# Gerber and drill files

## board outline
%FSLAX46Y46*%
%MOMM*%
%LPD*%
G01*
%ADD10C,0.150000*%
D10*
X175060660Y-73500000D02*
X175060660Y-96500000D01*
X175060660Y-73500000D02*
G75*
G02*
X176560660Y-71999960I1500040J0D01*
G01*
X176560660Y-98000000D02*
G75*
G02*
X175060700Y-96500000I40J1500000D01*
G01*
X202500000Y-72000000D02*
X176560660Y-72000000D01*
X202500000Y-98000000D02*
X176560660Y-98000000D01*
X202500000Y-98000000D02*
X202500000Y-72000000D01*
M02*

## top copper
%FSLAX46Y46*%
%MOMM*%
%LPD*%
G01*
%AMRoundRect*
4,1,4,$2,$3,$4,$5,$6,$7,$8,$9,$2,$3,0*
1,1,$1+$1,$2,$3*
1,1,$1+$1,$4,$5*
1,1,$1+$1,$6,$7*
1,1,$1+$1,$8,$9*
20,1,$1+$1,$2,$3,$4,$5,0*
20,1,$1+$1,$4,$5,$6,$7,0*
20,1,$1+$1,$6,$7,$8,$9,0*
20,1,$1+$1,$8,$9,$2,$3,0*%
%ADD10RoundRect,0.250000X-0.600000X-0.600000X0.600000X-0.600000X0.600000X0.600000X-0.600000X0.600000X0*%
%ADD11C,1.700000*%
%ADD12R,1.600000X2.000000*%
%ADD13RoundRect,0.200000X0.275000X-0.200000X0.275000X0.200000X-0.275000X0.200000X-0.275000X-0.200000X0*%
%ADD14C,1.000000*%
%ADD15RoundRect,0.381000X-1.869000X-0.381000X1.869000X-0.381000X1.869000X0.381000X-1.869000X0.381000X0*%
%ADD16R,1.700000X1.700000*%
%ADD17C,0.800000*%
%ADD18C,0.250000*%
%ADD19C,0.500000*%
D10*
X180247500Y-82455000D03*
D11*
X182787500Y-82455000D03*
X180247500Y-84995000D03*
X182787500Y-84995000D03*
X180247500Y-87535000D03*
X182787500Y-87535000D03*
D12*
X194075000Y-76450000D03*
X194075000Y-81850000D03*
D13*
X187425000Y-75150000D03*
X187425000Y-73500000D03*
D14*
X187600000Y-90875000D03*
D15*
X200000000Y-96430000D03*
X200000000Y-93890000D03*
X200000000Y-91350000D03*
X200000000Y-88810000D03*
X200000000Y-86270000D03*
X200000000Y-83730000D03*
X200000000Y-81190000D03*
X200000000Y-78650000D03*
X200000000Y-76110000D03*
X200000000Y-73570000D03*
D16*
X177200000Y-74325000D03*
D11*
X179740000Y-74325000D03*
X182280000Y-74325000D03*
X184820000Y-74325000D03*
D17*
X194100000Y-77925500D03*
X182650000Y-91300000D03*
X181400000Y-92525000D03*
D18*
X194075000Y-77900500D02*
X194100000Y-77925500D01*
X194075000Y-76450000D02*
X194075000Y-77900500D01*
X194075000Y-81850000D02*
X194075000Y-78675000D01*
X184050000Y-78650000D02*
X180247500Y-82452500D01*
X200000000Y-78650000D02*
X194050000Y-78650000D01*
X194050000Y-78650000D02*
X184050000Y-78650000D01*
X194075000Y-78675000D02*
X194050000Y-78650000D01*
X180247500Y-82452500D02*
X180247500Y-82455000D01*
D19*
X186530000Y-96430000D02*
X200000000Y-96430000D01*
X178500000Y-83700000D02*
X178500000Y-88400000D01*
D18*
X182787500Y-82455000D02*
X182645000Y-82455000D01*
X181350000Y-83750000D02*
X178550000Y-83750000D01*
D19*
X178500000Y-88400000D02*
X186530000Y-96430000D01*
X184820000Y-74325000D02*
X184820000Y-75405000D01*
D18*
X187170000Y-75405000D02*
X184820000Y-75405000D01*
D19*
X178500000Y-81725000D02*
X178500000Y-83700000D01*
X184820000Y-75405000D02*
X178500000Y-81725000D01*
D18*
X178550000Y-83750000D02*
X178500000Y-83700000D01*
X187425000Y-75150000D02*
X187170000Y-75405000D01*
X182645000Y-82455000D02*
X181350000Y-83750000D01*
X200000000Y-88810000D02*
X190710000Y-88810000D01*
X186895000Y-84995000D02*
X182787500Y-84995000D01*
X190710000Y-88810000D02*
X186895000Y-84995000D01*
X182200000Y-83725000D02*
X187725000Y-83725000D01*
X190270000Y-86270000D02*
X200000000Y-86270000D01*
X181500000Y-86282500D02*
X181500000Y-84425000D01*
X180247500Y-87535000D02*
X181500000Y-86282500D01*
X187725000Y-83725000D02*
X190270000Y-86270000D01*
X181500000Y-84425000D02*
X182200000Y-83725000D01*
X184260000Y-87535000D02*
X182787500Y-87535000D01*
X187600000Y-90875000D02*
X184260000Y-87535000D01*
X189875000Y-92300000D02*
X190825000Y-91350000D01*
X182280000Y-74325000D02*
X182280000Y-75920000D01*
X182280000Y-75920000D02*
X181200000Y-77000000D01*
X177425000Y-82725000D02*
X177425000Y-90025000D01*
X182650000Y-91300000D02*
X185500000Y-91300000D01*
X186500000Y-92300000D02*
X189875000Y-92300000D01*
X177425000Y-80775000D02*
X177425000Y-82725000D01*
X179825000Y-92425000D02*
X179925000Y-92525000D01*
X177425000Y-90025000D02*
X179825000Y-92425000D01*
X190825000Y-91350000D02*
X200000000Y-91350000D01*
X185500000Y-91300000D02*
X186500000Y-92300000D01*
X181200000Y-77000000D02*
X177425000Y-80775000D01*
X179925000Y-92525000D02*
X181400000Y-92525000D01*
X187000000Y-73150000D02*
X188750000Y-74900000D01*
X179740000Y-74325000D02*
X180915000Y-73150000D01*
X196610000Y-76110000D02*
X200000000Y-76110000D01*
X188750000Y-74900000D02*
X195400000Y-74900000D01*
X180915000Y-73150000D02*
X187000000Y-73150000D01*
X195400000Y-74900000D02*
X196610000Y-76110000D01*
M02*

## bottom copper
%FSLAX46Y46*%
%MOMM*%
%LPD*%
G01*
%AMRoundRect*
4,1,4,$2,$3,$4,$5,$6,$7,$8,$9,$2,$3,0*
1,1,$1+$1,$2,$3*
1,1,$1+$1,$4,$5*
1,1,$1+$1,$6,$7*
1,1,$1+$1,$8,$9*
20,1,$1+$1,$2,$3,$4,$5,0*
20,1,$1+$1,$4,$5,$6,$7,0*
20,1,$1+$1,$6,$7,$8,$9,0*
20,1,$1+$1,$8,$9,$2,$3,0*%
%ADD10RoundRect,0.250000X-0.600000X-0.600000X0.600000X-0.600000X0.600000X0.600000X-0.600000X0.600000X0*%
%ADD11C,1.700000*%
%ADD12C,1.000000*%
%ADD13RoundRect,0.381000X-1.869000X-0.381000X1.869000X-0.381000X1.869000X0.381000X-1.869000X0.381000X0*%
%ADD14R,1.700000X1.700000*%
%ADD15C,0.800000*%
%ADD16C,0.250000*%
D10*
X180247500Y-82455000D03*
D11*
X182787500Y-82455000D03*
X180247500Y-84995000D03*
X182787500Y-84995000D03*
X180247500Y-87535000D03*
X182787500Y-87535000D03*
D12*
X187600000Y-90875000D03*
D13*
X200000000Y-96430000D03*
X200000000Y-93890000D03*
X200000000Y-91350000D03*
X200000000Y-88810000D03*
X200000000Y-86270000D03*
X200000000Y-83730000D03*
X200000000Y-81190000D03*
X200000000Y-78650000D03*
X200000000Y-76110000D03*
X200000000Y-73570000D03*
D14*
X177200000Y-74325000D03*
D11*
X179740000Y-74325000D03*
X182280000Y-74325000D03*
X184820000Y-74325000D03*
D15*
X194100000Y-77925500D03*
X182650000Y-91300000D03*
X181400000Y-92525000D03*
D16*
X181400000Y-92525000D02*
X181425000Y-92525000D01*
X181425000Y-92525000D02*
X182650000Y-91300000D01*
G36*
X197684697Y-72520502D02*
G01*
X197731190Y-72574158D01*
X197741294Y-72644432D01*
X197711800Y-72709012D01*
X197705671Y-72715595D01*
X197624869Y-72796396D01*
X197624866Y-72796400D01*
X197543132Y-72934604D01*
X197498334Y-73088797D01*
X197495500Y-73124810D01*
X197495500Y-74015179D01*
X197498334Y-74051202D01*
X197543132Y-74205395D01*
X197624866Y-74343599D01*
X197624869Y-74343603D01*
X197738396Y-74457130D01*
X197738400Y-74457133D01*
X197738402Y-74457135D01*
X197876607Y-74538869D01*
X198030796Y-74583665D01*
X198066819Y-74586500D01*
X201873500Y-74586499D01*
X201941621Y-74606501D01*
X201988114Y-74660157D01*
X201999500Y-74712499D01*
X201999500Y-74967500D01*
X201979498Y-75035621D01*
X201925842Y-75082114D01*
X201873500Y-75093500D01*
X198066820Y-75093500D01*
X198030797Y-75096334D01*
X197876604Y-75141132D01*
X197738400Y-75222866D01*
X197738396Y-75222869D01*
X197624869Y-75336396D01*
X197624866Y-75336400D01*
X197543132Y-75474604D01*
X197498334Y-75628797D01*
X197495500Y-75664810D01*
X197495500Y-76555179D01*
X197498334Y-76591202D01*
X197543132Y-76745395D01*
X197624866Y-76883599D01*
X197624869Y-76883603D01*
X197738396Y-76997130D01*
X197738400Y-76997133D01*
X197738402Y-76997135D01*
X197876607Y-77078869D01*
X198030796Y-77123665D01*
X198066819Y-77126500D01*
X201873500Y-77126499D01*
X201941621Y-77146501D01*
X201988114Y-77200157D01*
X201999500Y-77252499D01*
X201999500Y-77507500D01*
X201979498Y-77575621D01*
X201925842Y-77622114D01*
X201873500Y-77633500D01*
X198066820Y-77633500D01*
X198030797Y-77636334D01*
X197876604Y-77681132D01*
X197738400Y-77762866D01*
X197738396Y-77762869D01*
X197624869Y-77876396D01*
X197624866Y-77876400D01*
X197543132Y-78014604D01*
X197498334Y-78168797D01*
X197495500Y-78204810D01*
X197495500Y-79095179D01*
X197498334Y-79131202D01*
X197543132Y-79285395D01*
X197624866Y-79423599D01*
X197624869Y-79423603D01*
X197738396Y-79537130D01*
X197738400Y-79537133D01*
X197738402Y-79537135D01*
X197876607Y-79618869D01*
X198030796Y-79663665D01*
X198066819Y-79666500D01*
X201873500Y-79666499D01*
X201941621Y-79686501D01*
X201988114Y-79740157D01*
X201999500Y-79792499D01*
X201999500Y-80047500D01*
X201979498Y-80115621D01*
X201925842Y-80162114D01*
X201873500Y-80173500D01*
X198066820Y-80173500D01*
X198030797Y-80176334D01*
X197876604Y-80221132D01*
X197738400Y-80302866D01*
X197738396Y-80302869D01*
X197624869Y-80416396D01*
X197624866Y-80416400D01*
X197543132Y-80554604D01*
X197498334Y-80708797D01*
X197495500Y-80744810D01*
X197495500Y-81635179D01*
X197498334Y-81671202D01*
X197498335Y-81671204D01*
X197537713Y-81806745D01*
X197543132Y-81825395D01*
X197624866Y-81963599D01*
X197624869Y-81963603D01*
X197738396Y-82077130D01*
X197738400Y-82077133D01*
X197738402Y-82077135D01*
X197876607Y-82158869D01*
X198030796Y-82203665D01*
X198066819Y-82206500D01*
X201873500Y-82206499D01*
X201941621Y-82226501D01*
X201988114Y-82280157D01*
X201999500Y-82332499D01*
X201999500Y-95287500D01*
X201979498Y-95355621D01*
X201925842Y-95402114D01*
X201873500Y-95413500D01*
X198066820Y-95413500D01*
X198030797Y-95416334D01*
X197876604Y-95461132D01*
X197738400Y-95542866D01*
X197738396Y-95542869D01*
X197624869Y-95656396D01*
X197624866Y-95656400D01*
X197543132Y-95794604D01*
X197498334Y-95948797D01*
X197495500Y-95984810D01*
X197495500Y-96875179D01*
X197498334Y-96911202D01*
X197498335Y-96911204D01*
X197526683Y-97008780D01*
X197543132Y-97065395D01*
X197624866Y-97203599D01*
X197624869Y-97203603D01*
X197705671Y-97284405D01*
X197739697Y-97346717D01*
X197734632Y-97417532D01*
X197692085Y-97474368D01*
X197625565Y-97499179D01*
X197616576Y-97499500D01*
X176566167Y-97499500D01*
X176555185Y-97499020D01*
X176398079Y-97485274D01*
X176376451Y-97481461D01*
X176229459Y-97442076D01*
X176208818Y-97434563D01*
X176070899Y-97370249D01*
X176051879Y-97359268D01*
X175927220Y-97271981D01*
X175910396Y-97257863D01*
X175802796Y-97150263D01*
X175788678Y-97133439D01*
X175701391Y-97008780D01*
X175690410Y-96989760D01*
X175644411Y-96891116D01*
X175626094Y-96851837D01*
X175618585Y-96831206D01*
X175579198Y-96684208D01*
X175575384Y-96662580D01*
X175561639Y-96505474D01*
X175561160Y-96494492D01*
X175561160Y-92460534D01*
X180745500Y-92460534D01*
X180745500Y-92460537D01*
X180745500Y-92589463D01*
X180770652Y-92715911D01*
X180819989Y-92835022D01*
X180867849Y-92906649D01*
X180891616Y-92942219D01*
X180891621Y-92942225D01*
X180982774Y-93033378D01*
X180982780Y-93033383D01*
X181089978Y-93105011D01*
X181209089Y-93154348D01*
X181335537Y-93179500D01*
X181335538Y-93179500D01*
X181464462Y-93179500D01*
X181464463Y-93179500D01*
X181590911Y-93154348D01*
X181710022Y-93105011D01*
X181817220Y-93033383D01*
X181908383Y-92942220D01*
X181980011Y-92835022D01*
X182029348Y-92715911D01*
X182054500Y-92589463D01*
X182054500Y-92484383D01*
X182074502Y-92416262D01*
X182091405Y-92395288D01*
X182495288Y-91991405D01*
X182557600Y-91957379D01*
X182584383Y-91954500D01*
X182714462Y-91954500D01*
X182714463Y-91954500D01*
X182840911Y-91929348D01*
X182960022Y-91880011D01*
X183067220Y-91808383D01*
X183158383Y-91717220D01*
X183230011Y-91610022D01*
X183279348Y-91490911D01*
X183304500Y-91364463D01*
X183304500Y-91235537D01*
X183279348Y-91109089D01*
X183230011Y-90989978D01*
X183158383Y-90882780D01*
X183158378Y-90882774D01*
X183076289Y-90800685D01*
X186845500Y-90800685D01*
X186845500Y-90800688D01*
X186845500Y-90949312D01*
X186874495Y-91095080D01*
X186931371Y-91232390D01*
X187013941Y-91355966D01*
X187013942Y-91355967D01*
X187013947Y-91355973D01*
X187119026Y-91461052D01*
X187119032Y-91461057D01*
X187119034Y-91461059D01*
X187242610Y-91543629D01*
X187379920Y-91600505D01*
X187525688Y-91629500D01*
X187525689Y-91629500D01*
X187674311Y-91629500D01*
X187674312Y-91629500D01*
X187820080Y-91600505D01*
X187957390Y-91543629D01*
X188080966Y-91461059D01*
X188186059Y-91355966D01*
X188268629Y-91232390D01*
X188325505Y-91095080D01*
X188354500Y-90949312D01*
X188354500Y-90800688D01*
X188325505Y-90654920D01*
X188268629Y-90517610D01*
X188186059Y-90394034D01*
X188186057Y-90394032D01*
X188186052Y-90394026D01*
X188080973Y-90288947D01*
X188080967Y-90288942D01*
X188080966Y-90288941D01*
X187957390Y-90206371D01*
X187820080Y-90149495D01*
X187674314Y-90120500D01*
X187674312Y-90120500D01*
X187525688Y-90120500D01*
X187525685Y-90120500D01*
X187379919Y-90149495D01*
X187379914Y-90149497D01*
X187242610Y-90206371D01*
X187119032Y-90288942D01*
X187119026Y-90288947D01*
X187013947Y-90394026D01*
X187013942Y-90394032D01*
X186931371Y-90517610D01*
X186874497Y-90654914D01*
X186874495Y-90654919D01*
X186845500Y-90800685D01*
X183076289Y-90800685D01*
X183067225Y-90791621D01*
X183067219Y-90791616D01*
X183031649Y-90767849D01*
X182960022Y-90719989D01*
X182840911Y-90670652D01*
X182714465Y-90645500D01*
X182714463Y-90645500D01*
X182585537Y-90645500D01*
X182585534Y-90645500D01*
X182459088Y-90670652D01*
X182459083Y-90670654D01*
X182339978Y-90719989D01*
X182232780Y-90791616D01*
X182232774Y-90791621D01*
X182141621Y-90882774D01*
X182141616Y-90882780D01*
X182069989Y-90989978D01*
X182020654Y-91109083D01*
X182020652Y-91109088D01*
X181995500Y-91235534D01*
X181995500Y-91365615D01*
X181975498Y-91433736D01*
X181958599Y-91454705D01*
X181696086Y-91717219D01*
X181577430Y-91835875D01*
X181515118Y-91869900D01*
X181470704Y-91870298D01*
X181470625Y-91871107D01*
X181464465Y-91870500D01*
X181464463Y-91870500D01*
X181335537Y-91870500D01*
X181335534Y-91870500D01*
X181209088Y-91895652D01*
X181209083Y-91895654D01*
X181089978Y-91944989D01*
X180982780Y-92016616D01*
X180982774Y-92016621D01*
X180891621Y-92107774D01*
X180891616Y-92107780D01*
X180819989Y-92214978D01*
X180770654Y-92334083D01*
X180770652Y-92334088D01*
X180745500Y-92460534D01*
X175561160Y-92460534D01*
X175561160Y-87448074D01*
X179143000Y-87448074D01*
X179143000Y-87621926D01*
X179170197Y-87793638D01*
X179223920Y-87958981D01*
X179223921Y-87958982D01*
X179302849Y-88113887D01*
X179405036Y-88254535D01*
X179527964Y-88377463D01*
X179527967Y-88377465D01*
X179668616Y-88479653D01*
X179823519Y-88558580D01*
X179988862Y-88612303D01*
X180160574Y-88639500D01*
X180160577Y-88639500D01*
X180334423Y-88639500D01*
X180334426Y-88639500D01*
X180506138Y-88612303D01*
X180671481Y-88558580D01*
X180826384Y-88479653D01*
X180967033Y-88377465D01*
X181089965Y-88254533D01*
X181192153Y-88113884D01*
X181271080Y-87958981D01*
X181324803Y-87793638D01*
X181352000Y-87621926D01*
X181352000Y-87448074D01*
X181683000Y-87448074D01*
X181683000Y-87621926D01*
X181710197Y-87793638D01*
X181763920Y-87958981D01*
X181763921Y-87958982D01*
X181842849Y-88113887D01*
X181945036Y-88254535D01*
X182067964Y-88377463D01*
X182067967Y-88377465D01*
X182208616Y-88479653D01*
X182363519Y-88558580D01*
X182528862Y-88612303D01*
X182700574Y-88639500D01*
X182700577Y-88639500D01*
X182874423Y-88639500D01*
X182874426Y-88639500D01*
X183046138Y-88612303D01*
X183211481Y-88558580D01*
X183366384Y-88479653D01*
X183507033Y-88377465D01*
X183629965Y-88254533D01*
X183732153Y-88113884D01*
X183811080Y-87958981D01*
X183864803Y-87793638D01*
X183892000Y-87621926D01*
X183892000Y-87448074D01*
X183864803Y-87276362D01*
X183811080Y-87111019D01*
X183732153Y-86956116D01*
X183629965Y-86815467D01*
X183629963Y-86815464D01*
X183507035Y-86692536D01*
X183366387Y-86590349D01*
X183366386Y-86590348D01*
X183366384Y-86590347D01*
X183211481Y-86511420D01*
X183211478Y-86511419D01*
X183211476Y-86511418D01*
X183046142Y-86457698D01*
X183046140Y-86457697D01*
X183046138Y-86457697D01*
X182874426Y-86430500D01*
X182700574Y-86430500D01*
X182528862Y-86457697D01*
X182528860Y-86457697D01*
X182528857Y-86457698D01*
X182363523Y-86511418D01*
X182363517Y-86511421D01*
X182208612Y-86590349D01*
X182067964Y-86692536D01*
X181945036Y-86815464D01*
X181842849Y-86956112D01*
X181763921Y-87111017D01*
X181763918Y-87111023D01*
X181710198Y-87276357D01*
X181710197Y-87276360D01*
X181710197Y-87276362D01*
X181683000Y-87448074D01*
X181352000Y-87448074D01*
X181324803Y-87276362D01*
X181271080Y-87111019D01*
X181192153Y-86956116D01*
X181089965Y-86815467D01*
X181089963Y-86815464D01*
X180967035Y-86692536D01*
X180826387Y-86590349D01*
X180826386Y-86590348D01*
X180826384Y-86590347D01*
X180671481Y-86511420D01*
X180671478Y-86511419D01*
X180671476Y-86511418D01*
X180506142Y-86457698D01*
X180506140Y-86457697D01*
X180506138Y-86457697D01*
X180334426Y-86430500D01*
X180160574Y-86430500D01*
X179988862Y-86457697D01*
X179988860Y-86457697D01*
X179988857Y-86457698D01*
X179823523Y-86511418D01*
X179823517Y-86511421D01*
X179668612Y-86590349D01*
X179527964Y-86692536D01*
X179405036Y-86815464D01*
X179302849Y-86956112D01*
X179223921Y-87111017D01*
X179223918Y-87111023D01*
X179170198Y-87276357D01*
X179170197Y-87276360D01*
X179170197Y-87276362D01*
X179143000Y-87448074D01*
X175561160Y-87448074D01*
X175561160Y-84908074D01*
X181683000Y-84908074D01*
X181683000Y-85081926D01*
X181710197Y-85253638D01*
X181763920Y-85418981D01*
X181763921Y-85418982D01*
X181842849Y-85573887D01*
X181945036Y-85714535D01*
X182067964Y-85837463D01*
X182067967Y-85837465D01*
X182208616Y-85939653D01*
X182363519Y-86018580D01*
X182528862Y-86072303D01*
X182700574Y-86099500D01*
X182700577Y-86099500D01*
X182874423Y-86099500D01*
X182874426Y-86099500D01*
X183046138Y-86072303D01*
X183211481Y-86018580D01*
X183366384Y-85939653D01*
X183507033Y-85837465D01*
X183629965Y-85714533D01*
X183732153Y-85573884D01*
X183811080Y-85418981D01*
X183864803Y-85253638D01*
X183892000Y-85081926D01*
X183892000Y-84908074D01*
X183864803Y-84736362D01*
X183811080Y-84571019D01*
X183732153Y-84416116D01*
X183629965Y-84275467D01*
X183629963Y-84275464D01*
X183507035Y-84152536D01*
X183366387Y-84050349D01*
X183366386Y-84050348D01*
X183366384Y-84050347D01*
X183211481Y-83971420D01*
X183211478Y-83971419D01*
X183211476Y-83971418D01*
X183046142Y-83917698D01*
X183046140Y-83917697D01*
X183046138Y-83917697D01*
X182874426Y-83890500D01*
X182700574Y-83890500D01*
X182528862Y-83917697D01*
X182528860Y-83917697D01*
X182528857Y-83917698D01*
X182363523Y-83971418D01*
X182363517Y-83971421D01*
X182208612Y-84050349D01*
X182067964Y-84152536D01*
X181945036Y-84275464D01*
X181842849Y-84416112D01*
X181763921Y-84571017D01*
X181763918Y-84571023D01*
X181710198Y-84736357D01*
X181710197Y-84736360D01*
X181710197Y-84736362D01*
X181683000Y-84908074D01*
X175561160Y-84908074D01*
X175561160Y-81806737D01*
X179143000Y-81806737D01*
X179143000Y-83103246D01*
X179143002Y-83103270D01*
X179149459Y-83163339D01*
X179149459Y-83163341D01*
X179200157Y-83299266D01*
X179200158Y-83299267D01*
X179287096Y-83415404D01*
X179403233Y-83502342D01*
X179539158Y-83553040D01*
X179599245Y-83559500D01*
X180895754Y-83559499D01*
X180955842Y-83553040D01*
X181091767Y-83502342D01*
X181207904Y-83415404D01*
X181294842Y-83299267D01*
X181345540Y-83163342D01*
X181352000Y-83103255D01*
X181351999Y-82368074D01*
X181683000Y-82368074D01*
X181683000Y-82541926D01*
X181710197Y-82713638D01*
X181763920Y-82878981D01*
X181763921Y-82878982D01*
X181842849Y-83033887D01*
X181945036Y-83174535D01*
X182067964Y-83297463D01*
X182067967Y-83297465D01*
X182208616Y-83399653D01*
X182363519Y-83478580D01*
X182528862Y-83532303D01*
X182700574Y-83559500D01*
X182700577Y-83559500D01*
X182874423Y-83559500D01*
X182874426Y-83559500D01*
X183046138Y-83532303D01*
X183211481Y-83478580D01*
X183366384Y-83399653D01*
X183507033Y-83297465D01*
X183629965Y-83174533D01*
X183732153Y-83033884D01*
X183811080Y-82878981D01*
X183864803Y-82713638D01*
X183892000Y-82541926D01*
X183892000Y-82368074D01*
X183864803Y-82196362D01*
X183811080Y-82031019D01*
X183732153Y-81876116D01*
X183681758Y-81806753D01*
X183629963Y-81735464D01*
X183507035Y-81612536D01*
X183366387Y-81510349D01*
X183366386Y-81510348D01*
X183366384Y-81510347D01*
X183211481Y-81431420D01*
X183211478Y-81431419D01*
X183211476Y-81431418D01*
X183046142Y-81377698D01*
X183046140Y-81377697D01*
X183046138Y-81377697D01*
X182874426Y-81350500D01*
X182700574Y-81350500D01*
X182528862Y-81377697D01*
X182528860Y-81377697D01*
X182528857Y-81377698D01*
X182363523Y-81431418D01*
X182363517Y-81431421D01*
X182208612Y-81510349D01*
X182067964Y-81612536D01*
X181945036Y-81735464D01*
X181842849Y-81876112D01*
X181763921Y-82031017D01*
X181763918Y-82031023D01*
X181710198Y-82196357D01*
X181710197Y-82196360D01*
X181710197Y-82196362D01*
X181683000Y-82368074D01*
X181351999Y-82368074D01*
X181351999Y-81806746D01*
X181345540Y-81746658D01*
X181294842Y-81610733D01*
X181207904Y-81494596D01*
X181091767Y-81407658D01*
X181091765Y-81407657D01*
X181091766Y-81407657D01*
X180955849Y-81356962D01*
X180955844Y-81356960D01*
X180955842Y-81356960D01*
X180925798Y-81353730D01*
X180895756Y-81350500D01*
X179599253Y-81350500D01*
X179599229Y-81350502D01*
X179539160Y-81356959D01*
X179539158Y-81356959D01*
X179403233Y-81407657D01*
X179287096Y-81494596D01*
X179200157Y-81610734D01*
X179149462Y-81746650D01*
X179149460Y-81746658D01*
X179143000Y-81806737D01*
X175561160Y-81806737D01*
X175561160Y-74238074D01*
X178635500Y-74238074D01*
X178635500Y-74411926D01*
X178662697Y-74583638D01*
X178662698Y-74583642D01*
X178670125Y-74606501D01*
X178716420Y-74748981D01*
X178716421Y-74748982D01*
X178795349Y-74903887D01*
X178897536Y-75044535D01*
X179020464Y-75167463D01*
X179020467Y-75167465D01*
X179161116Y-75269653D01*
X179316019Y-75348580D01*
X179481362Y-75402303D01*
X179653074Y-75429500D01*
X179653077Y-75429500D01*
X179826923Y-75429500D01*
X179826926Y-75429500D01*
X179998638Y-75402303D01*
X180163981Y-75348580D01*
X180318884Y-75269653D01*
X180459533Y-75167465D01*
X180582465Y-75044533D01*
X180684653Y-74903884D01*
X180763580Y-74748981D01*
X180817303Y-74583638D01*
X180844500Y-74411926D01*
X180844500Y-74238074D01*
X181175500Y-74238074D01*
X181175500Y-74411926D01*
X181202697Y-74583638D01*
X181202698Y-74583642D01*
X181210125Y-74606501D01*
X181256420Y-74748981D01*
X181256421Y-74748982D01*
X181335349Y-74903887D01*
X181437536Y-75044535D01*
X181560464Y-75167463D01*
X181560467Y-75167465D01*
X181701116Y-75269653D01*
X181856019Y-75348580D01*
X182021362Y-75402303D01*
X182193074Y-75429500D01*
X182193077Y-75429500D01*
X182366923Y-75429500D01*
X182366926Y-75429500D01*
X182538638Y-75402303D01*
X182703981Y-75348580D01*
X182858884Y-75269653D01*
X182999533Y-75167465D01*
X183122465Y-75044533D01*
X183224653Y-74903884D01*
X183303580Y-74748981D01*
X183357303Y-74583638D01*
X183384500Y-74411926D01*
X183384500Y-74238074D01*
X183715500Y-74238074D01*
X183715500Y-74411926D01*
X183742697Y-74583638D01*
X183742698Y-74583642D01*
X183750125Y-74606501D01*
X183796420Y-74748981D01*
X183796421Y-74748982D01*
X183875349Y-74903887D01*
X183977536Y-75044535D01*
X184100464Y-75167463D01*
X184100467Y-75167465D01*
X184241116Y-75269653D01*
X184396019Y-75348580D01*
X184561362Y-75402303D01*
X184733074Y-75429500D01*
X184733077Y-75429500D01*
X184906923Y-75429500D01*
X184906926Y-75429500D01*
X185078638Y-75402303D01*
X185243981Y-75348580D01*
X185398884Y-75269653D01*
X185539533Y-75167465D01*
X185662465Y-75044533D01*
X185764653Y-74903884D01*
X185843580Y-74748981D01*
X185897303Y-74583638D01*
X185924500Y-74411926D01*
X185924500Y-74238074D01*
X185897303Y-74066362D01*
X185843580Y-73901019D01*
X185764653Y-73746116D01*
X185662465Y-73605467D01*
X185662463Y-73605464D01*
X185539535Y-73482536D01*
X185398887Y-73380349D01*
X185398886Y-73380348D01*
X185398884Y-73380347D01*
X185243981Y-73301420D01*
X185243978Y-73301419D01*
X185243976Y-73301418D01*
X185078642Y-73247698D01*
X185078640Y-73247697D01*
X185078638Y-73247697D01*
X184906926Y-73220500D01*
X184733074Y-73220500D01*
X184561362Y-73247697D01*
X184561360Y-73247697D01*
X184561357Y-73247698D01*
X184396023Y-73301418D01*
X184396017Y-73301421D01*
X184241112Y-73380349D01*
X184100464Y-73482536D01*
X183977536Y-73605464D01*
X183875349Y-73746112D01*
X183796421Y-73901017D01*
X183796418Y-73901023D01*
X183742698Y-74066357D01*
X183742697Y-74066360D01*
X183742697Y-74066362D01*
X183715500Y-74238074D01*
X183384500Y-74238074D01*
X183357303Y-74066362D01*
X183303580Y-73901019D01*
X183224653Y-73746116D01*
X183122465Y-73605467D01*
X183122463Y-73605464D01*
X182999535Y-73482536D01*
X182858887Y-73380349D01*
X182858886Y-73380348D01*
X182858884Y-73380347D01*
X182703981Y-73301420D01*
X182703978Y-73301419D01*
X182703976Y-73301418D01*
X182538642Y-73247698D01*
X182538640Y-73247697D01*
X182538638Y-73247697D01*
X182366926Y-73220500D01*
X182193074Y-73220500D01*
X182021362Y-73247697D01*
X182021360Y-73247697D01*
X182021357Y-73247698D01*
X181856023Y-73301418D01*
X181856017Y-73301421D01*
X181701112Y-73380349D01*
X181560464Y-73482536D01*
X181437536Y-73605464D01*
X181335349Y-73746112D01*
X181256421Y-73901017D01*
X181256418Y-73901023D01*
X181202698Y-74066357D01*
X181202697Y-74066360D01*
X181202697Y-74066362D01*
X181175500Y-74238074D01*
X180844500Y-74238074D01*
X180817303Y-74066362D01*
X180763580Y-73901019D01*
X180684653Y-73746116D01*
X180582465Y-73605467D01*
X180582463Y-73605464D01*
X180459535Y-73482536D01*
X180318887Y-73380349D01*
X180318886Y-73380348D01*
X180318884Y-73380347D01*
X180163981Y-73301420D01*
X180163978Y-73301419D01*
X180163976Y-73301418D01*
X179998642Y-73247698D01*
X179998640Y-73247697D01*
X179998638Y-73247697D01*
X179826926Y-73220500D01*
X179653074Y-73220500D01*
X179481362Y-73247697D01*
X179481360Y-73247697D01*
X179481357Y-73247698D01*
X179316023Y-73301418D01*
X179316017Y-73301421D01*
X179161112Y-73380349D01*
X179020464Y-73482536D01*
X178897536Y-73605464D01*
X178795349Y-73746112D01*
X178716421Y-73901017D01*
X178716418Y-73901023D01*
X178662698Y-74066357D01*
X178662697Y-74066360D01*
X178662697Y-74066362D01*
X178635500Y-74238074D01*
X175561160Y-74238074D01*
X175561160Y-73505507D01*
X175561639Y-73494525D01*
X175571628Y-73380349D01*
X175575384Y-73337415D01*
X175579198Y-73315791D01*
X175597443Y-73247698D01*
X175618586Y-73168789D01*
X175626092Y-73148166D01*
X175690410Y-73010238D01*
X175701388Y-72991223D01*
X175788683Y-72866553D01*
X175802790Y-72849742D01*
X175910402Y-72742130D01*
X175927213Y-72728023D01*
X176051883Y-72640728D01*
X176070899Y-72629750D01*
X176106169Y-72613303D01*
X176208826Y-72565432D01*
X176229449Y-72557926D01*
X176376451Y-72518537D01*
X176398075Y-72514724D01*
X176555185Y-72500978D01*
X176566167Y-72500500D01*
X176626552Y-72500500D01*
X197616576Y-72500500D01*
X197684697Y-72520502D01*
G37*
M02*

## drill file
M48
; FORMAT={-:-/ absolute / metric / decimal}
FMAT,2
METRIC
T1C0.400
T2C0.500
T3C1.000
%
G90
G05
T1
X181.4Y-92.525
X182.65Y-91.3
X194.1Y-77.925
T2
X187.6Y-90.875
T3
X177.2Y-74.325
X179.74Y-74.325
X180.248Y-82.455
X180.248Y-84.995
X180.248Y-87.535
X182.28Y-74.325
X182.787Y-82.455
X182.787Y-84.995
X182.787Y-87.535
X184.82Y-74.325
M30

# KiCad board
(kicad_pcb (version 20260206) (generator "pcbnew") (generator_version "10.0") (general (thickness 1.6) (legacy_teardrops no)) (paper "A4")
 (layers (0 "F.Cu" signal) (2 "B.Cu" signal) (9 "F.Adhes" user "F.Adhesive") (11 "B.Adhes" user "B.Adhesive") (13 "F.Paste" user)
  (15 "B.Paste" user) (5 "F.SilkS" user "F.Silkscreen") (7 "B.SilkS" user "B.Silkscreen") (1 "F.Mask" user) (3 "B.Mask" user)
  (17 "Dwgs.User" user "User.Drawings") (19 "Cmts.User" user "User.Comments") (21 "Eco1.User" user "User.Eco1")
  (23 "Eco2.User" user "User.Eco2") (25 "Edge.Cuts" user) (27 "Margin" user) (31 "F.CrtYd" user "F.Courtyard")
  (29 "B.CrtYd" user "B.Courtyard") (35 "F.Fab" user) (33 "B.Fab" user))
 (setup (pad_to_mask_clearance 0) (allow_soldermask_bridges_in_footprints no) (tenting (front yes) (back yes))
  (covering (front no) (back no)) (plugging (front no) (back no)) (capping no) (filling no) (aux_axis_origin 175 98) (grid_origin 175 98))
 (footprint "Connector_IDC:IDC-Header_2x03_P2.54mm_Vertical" (layer "F.Cu") (at 180.2475 82.455)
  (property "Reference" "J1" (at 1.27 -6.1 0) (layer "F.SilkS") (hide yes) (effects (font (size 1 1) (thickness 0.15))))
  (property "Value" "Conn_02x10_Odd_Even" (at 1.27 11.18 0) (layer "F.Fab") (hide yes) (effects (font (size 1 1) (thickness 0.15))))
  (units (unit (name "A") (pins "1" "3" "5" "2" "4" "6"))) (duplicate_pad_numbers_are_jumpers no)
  (pad "1" thru_hole roundrect (at 0 0) (size 1.7 1.7) (drill 1) (layers "*.Cu" "*.Mask") (remove_unused_layers no)
   (roundrect_rratio 0.147059) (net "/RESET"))
  (pad "2" thru_hole circle (at 2.54 0) (size 1.7 1.7) (drill 1) (layers "*.Cu" "*.Mask") (remove_unused_layers no) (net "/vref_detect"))
  (pad "3" thru_hole circle (at 0 2.54) (size 1.7 1.7) (drill 1) (layers "*.Cu" "*.Mask") (remove_unused_layers no) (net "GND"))
  (pad "4" thru_hole circle (at 2.54 2.54) (size 1.7 1.7) (drill 1) (layers "*.Cu" "*.Mask") (remove_unused_layers no) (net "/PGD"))
  (pad "5" thru_hole circle (at 0 5.08) (size 1.7 1.7) (drill 1) (layers "*.Cu" "*.Mask") (remove_unused_layers no) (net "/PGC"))
  (pad "6" thru_hole circle (at 2.54 5.08) (size 1.7 1.7) (drill 1) (layers "*.Cu" "*.Mask") (remove_unused_layers no) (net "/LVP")))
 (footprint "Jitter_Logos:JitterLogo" (layer "F.Cu") (at 193.607667 90.975)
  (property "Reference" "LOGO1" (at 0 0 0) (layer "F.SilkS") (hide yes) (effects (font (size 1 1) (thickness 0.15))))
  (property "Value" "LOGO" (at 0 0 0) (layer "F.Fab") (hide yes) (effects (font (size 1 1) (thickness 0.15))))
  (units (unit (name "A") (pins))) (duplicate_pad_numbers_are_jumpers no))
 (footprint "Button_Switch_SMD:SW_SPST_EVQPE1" (layer "F.Cu") (at 194.075 79.15 -90)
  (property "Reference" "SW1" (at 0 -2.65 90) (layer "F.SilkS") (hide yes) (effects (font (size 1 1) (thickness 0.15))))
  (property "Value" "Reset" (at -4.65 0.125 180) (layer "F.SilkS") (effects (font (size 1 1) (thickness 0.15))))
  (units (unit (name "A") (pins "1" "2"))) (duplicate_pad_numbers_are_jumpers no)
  (pad "1" smd rect (at -2.7 0 270) (size 2 1.6) (layers "F.Cu" "F.Mask" "F.Paste") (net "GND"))
  (pad "2" smd rect (at 2.7 0 270) (size 2 1.6) (layers "F.Cu" "F.Mask" "F.Paste") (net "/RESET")))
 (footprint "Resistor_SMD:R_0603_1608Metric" (layer "F.Cu") (at 187.425 74.325 90)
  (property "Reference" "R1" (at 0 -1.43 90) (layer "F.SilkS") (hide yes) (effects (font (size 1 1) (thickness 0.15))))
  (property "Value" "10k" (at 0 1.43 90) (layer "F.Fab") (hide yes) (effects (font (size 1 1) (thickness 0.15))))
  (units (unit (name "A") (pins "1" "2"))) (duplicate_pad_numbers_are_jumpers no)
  (pad "1" smd roundrect (at -0.825 0 90) (size 0.8 0.95) (layers "F.Cu" "F.Mask" "F.Paste") (roundrect_rratio 0.25) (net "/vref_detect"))
  (pad "2" smd roundrect (at 0.825 0 90) (size 0.8 0.95) (layers "F.Cu" "F.Mask" "F.Paste") (roundrect_rratio 0.25) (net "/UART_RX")))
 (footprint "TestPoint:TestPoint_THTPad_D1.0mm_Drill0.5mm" (layer "F.Cu") (at 187.6 90.875)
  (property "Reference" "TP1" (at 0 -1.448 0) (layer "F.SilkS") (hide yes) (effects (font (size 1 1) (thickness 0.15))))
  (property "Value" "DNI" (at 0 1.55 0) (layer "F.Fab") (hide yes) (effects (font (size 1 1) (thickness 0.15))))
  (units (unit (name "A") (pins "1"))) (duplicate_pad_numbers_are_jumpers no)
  (pad "1" thru_hole circle (at 0 0) (size 1 1) (drill 0.5) (layers "*.Cu" "*.Mask") (remove_unused_layers no) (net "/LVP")))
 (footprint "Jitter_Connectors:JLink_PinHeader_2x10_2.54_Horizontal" (layer "F.Cu") (at 200 85)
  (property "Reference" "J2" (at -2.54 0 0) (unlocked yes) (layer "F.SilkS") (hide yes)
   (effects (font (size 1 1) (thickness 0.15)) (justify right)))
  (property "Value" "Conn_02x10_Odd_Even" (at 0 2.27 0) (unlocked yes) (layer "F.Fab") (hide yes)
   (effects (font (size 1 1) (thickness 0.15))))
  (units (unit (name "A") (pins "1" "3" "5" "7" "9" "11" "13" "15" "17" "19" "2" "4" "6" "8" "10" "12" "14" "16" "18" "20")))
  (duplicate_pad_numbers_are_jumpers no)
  (pad "1" smd roundrect (at 0 11.43) (size 4.5 1.524) (layers "F.Cu" "F.Mask" "F.Paste") (roundrect_rratio 0.25) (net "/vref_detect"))
  (pad "2" smd roundrect (at 0 11.43) (size 4.5 1.524) (layers "B.Cu" "B.Mask" "B.Paste") (roundrect_rratio 0.25)
   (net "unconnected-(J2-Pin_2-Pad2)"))
  (pad "3" smd roundrect (at 0 8.89) (size 4.5 1.524) (layers "F.Cu" "F.Mask" "F.Paste") (roundrect_rratio 0.25)
   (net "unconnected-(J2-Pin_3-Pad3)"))
  (pad "4" smd roundrect (at 0 8.89) (size 4.5 1.524) (layers "B.Cu" "B.Mask" "B.Paste") (roundrect_rratio 0.25) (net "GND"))
  (pad "5" smd roundrect (at 0 6.35) (size 4.5 1.524) (layers "F.Cu" "F.Mask" "F.Paste") (roundrect_rratio 0.25) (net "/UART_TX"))
  (pad "6" smd roundrect (at 0 6.35) (size 4.5 1.524) (layers "B.Cu" "B.Mask" "B.Paste") (roundrect_rratio 0.25) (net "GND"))
  (pad "7" smd roundrect (at 0 3.81) (size 4.5 1.524) (layers "F.Cu" "F.Mask" "F.Paste") (roundrect_rratio 0.25) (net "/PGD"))
  (pad "8" smd roundrect (at 0 3.81) (size 4.5 1.524) (layers "B.Cu" "B.Mask" "B.Paste") (roundrect_rratio 0.25) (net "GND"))
  (pad "9" smd roundrect (at 0 1.27) (size 4.5 1.524) (layers "F.Cu" "F.Mask" "F.Paste") (roundrect_rratio 0.25) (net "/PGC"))
  (pad "10" smd roundrect (at 0 1.27) (size 4.5 1.524) (layers "B.Cu" "B.Mask" "B.Paste") (roundrect_rratio 0.25) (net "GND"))
  (pad "11" smd roundrect (at 0 -1.27) (size 4.5 1.524) (layers "F.Cu" "F.Mask" "F.Paste") (roundrect_rratio 0.25)
   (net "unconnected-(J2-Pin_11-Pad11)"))
  (pad "12" smd roundrect (at 0 -1.27) (size 4.5 1.524) (layers "B.Cu" "B.Mask" "B.Paste") (roundrect_rratio 0.25) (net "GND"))
  (pad "13" smd roundrect (at 0 -3.81) (size 4.5 1.524) (layers "F.Cu" "F.Mask" "F.Paste") (roundrect_rratio 0.25)
   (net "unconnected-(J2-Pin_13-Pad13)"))
  (pad "14" smd roundrect (at 0 -3.81) (size 4.5 1.524) (layers "B.Cu" "B.Mask" "B.Paste") (roundrect_rratio 0.25)
   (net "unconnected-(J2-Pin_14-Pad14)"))
  (pad "15" smd roundrect (at 0 -6.35) (size 4.5 1.524) (layers "F.Cu" "F.Mask" "F.Paste") (roundrect_rratio 0.25) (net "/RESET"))
  (pad "16" smd roundrect (at 0 -6.35) (size 4.5 1.524) (layers "B.Cu" "B.Mask" "B.Paste") (roundrect_rratio 0.25)
   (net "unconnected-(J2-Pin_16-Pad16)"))
  (pad "17" smd roundrect (at 0 -8.89) (size 4.5 1.524) (layers "F.Cu" "F.Mask" "F.Paste") (roundrect_rratio 0.25) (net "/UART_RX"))
  (pad "18" smd roundrect (at 0 -8.89) (size 4.5 1.524) (layers "B.Cu" "B.Mask" "B.Paste") (roundrect_rratio 0.25)
   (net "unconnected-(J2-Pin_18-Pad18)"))
  (pad "19" smd roundrect (at 0 -11.43) (size 4.5 1.524) (layers "F.Cu" "F.Mask" "F.Paste") (roundrect_rratio 0.25)
   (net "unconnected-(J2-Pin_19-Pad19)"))
  (pad "20" smd roundrect (at 0 -11.43) (size 4.5 1.524) (layers "B.Cu" "B.Mask" "B.Paste") (roundrect_rratio 0.25)
   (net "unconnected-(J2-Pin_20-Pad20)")))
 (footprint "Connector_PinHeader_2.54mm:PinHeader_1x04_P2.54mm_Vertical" (layer "F.Cu") (at 177.2 74.325 90)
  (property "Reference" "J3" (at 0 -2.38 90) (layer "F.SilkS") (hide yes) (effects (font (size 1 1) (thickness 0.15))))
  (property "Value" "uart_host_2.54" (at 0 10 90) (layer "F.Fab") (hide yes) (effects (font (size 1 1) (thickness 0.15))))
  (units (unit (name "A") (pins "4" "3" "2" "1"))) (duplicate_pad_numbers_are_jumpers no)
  (pad "1" thru_hole rect (at 0 0 90) (size 1.7 1.7) (drill 1) (layers "*.Cu" "*.Mask") (remove_unused_layers no) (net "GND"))
  (pad "2" thru_hole circle (at 0 2.54 90) (size 1.7 1.7) (drill 1) (layers "*.Cu" "*.Mask") (remove_unused_layers no) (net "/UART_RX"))
  (pad "3" thru_hole circle (at 0 5.08 90) (size 1.7 1.7) (drill 1) (layers "*.Cu" "*.Mask") (remove_unused_layers no) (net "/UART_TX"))
  (pad "4" thru_hole circle (at 0 7.62 90) (size 1.7 1.7) (drill 1) (layers "*.Cu" "*.Mask") (remove_unused_layers no) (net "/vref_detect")))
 (gr_line (start 175.06066 73.5) (end 175.06066 96.5) (stroke (width 0.15) (type solid)) (layer "Edge.Cuts"))
 (gr_arc (start 175.06066 73.5) (mid 175.5 72.43934) (end 176.56066 72) (stroke (width 0.15) (type solid)) (layer "Edge.Cuts"))
 (gr_arc (start 176.56066 98) (mid 175.5 97.56066) (end 175.06066 96.5) (stroke (width 0.15) (type solid)) (layer "Edge.Cuts"))
 (gr_line (start 202.5 72) (end 176.56066 72) (stroke (width 0.15) (type solid)) (layer "Edge.Cuts"))
 (gr_line (start 202.5 98) (end 176.56066 98) (stroke (width 0.15) (type solid)) (layer "Edge.Cuts"))
 (gr_line (start 202.5 98) (end 202.5 72) (stroke (width 0.15) (type solid)) (layer "Edge.Cuts"))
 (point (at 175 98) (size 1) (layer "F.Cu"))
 (segment (start 194.075 77.9005) (end 194.1 77.9255) (width 0.25) (layer "F.Cu") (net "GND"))
 (segment (start 194.075 76.45) (end 194.075 77.9005) (width 0.25) (layer "F.Cu") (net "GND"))
 (via (at 194.1 77.9255) (size 0.8) (drill 0.4) (layers "F.Cu" "B.Cu") (capping no) (covering (front no) (back no))
  (plugging (front no) (back no)) (filling no) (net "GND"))
 (segment (start 194.075 81.85) (end 194.075 78.675) (width 0.25) (layer "F.Cu") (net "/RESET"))
 (segment (start 184.05 78.65) (end 180.2475 82.4525) (width 0.25) (layer "F.Cu") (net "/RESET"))
 (segment (start 200 78.65) (end 194.05 78.65) (width 0.25) (layer "F.Cu") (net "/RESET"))
 (segment (start 194.05 78.65) (end 184.05 78.65) (width 0.25) (layer "F.Cu") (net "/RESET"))
 (segment (start 194.075 78.675) (end 194.05 78.65) (width 0.25) (layer "F.Cu") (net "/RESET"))
 (segment (start 180.2475 82.4525) (end 180.2475 82.455) (width 0.25) (layer "F.Cu") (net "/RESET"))
 (segment (start 186.53 96.43) (end 200 96.43) (width 0.5) (layer "F.Cu") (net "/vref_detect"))
 (segment (start 178.5 83.7) (end 178.5 88.4) (width 0.5) (layer "F.Cu") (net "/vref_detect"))
 (segment (start 182.7875 82.455) (end 182.645 82.455) (width 0.25) (layer "F.Cu") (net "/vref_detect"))
 (segment (start 181.35 83.75) (end 178.55 83.75) (width 0.25) (layer "F.Cu") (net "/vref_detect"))
 (segment (start 178.5 88.4) (end 186.53 96.43) (width 0.5) (layer "F.Cu") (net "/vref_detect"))
 (segment (start 184.82 74.325) (end 184.82 75.405) (width 0.5) (layer "F.Cu") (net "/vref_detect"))
 (segment (start 187.17 75.405) (end 184.82 75.405) (width 0.25) (layer "F.Cu") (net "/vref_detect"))
 (segment (start 178.5 81.725) (end 178.5 83.7) (width 0.5) (layer "F.Cu") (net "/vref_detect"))
 (segment (start 184.82 75.405) (end 178.5 81.725) (width 0.5) (layer "F.Cu") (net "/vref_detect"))
 (segment (start 178.55 83.75) (end 178.5 83.7) (width 0.25) (layer "F.Cu") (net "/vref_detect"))
 (segment (start 187.425 75.15) (end 187.17 75.405) (width 0.25) (layer "F.Cu") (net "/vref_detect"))
 (segment (start 182.645 82.455) (end 181.35 83.75) (width 0.25) (layer "F.Cu") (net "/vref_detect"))
 (segment (start 200 88.81) (end 190.71 88.81) (width 0.25) (layer "F.Cu") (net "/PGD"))
 (segment (start 186.895 84.995) (end 182.7875 84.995) (width 0.25) (layer "F.Cu") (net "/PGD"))
 (segment (start 190.71 88.81) (end 186.895 84.995) (width 0.25) (layer "F.Cu") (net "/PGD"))
 (segment (start 182.2 83.725) (end 187.725 83.725) (width 0.25) (layer "F.Cu") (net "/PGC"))
 (segment (start 190.27 86.27) (end 200 86.27) (width 0.25) (layer "F.Cu") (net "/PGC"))
 (segment (start 181.5 86.2825) (end 181.5 84.425) (width 0.25) (layer "F.Cu") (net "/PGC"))
 (segment (start 180.2475 87.535) (end 181.5 86.2825) (width 0.25) (layer "F.Cu") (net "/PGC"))
 (segment (start 187.725 83.725) (end 190.27 86.27) (width 0.25) (layer "F.Cu") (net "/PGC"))
 (segment (start 181.5 84.425) (end 182.2 83.725) (width 0.25) (layer "F.Cu") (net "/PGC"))
 (segment (start 184.26 87.535) (end 182.7875 87.535) (width 0.25) (layer "F.Cu") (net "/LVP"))
 (segment (start 187.6 90.875) (end 184.26 87.535) (width 0.25) (layer "F.Cu") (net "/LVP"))
 (segment (start 189.875 92.3) (end 190.825 91.35) (width 0.25) (layer "F.Cu") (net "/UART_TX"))
 (segment (start 182.28 74.325) (end 182.28 75.92) (width 0.25) (layer "F.Cu") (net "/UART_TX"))
 (segment (start 182.28 75.92) (end 181.2 77) (width 0.25) (layer "F.Cu") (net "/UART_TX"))
 (segment (start 177.425 82.725) (end 177.425 90.025) (width 0.25) (layer "F.Cu") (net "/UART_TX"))
 (segment (start 182.65 91.3) (end 185.5 91.3) (width 0.25) (layer "F.Cu") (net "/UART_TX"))
 (segment (start 186.5 92.3) (end 189.875 92.3) (width 0.25) (layer "F.Cu") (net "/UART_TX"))
 (segment (start 177.425 80.775) (end 177.425 82.725) (width 0.25) (layer "F.Cu") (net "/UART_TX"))
 (segment (start 179.825 92.425) (end 179.925 92.525) (width 0.25) (layer "F.Cu") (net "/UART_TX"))
 (segment (start 177.425 90.025) (end 179.825 92.425) (width 0.25) (layer "F.Cu") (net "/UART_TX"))
 (segment (start 190.825 91.35) (end 200 91.35) (width 0.25) (layer "F.Cu") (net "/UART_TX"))
 (segment (start 185.5 91.3) (end 186.5 92.3) (width 0.25) (layer "F.Cu") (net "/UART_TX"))
 (segment (start 181.2 77) (end 177.425 80.775) (width 0.25) (layer "F.Cu") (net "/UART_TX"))
 (segment (start 179.925 92.525) (end 181.4 92.525) (width 0.25) (layer "F.Cu") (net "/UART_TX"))
 (via (at 182.65 91.3) (size 0.8) (drill 0.4) (layers "F.Cu" "B.Cu") (capping no) (covering (front no) (back no))
  (plugging (front no) (back no)) (filling no) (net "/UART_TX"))
 (via (at 181.4 92.525) (size 0.8) (drill 0.4) (layers "F.Cu" "B.Cu") (capping no) (covering (front no) (back no))
  (plugging (front no) (back no)) (filling no) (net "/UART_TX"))
 (segment (start 181.4 92.525) (end 181.425 92.525) (width 0.25) (layer "B.Cu") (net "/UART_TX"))
 (segment (start 181.425 92.525) (end 182.65 91.3) (width 0.25) (layer "B.Cu") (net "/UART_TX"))
 (segment (start 187 73.15) (end 188.75 74.9) (width 0.25) (layer "F.Cu") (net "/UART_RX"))
 (segment (start 179.74 74.325) (end 180.915 73.15) (width 0.25) (layer "F.Cu") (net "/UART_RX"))
 (segment (start 196.61 76.11) (end 200 76.11) (width 0.25) (layer "F.Cu") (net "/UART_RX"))
 (segment (start 188.75 74.9) (end 195.4 74.9) (width 0.25) (layer "F.Cu") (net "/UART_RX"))
 (segment (start 180.915 73.15) (end 187 73.15) (width 0.25) (layer "F.Cu") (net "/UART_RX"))
 (segment (start 195.4 74.9) (end 196.61 76.11) (width 0.25) (layer "F.Cu") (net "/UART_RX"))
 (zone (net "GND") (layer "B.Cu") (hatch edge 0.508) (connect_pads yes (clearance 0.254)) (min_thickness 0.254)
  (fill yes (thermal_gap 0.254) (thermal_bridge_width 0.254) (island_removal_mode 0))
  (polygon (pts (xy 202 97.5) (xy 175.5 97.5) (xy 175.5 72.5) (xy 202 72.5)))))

